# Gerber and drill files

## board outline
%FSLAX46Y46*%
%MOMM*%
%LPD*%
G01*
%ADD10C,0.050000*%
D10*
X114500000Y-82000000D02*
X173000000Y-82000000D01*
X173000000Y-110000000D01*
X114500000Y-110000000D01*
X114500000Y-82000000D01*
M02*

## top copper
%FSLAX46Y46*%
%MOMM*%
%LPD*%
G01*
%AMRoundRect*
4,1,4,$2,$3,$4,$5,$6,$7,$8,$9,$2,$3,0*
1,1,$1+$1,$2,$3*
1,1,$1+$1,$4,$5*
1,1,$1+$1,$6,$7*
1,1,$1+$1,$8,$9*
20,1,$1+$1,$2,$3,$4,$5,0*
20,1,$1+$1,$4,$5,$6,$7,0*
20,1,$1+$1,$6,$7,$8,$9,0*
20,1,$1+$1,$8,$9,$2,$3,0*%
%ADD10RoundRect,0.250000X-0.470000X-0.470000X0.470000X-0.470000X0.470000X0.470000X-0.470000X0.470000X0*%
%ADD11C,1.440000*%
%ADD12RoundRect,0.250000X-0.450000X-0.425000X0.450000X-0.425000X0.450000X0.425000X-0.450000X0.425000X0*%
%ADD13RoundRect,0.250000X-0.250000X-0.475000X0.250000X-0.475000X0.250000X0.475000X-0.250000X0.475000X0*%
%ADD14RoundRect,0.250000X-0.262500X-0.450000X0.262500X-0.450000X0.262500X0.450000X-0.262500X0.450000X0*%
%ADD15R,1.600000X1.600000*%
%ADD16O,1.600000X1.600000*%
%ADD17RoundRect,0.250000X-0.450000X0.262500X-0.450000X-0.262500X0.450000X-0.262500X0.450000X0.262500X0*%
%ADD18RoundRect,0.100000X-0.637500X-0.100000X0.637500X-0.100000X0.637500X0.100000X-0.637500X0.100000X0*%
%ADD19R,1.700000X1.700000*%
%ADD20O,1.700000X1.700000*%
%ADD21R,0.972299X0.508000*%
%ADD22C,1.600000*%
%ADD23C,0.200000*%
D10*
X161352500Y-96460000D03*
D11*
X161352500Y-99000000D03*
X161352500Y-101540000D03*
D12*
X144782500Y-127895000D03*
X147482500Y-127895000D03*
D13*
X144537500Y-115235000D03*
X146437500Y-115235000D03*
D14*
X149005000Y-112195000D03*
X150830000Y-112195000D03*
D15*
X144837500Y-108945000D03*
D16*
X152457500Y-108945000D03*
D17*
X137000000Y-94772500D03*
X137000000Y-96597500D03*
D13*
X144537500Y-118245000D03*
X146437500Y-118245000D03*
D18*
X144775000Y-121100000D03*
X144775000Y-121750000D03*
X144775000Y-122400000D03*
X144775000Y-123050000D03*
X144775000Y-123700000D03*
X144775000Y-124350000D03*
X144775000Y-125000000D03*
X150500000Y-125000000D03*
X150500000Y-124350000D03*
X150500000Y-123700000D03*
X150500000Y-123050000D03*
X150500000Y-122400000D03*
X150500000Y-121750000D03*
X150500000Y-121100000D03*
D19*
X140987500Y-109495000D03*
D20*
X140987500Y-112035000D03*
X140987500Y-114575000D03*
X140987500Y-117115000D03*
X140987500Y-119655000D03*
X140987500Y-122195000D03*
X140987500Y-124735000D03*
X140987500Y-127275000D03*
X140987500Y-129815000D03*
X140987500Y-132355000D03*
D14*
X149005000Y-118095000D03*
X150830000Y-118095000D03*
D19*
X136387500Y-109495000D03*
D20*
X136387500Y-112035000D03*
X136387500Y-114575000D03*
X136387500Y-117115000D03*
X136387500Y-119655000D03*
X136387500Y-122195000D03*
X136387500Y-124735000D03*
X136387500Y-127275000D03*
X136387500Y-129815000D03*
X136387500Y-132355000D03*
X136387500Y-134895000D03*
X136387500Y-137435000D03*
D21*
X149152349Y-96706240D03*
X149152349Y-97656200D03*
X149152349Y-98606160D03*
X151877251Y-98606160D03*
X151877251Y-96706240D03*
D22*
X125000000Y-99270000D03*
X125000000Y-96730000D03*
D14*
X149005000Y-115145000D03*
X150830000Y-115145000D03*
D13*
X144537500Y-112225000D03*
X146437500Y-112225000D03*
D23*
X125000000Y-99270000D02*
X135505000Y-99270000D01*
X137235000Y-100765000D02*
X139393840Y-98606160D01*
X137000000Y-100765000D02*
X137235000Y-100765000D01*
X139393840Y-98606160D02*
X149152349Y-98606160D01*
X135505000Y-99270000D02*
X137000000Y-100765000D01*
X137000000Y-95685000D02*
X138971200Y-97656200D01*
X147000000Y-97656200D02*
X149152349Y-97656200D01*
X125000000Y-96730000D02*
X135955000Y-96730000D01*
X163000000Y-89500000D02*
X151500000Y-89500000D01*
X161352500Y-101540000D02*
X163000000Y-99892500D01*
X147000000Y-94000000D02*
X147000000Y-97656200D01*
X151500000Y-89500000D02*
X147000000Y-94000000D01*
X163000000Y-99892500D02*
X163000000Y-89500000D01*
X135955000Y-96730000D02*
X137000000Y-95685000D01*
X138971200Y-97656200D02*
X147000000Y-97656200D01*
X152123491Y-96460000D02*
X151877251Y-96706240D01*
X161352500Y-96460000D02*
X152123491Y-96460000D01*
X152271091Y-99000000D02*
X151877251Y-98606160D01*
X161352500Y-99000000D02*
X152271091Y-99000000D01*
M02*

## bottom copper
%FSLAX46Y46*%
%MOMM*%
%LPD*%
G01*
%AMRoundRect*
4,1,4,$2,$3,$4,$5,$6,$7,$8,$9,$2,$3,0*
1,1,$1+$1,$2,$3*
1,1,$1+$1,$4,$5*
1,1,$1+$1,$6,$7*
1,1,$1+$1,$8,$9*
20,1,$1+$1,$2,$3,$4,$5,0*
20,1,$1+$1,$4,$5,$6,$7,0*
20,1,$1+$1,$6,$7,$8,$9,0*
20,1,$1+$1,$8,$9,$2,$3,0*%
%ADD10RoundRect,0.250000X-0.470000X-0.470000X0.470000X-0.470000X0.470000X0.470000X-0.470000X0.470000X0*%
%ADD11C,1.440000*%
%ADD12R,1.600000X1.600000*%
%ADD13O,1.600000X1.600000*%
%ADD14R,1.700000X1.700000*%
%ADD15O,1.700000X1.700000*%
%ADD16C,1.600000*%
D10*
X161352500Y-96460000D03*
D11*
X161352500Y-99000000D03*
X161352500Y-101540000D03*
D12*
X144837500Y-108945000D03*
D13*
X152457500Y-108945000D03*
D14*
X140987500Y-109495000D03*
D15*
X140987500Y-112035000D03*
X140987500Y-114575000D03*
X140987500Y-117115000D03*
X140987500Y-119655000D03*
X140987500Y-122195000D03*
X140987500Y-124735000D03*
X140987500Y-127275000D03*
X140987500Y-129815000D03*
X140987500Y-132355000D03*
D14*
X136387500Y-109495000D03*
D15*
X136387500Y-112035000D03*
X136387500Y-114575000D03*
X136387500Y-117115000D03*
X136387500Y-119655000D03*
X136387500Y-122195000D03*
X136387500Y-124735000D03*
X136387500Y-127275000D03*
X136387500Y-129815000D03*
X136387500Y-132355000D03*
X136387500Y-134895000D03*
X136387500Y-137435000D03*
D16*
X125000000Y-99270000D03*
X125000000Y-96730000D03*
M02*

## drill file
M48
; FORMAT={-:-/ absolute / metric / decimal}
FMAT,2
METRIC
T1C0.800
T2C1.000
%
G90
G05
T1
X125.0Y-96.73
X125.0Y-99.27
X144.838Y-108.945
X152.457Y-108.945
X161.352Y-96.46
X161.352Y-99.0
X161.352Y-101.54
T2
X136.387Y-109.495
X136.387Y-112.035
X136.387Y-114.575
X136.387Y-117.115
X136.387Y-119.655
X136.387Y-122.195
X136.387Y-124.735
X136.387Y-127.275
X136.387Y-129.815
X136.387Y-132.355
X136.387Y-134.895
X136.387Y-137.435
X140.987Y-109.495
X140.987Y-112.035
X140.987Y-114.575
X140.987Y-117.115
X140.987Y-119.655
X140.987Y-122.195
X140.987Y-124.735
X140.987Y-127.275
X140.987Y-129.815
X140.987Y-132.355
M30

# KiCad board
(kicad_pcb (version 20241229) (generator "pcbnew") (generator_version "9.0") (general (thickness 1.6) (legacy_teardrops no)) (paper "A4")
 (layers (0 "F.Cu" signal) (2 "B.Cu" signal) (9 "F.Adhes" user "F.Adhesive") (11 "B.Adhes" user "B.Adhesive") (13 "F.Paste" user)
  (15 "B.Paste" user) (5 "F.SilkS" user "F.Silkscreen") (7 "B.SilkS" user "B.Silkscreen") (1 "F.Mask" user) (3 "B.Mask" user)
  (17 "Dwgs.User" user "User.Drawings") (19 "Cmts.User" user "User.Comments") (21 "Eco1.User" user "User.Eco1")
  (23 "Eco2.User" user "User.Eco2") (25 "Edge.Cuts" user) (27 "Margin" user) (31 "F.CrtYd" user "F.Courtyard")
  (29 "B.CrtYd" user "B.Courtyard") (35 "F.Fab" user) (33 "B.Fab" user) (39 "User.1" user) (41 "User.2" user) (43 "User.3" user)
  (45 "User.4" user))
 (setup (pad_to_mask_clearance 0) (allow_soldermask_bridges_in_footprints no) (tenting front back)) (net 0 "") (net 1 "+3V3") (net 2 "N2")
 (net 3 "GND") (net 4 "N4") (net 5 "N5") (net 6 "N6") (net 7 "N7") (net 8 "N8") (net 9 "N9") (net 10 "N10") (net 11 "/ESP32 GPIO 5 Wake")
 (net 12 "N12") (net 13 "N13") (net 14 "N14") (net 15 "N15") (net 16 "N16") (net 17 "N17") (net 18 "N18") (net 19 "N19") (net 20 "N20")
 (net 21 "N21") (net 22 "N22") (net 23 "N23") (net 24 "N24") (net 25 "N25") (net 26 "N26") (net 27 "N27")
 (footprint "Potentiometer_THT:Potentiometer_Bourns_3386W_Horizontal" (layer "F.Cu") (at 161.3525 96.46 -90)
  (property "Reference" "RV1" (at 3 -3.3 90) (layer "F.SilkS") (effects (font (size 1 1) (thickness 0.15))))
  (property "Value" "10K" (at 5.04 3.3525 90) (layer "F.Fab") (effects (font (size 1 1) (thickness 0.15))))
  (pad "1" thru_hole roundrect (at 0 0) (size 1.44 1.44) (drill 0.8) (layers "*.Cu" "*.Mask") (remove_unused_layers no)
   (roundrect_rratio 0.1736111111) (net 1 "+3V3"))
  (pad "2" thru_hole circle (at 2.54 0) (size 1.44 1.44) (drill 0.8) (layers "*.Cu" "*.Mask") (remove_unused_layers no) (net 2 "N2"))
  (pad "3" thru_hole circle (at 5.08 0) (size 1.44 1.44) (drill 0.8) (layers "*.Cu" "*.Mask") (remove_unused_layers no) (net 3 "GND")))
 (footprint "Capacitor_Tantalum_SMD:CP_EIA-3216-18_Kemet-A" (layer "F.Cu") (at 146.1325 127.895)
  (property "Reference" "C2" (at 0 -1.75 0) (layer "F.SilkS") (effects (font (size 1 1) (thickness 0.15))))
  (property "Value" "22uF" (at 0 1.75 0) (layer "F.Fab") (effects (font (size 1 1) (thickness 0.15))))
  (pad "1" smd roundrect (at -1.35 0) (size 1.4 1.35) (layers "F.Cu" "F.Mask" "F.Paste") (roundrect_rratio 0.185185) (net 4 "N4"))
  (pad "2" smd roundrect (at 1.35 0) (size 1.4 1.35) (layers "F.Cu" "F.Mask" "F.Paste") (roundrect_rratio 0.185185) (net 3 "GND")))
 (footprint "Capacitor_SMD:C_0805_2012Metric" (layer "F.Cu") (at 145.4875 115.235)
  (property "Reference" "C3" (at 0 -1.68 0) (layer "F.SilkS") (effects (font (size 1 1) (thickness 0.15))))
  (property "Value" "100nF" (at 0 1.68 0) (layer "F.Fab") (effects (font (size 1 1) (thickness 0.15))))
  (pad "1" smd roundrect (at -0.95 0) (size 1 1.45) (layers "F.Cu" "F.Mask" "F.Paste") (roundrect_rratio 0.25) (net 1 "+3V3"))
  (pad "2" smd roundrect (at 0.95 0) (size 1 1.45) (layers "F.Cu" "F.Mask" "F.Paste") (roundrect_rratio 0.25) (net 3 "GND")))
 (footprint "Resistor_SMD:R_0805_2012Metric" (layer "F.Cu") (at 149.9175 112.195)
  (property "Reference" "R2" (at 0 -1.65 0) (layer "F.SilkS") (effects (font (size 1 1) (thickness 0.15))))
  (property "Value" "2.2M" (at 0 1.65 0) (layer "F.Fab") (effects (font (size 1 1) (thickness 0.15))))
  (pad "1" smd roundrect (at -0.9125 0) (size 1.025 1.4) (layers "F.Cu" "F.Mask" "F.Paste") (roundrect_rratio 0.243902) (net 4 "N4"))
  (pad "2" smd roundrect (at 0.9125 0) (size 1.025 1.4) (layers "F.Cu" "F.Mask" "F.Paste") (roundrect_rratio 0.243902) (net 1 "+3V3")))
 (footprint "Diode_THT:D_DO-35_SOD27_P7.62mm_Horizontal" (layer "F.Cu") (at 144.8375 108.945)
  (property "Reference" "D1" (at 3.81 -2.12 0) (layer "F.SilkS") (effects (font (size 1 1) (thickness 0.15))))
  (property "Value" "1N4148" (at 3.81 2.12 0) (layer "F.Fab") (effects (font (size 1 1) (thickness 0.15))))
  (pad "1" thru_hole rect (at 0 0) (size 1.6 1.6) (drill 0.8) (layers "*.Cu" "*.Mask") (remove_unused_layers no) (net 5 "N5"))
  (pad "2" thru_hole oval (at 7.62 0) (size 1.6 1.6) (drill 0.8) (layers "*.Cu" "*.Mask") (remove_unused_layers no) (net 4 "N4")))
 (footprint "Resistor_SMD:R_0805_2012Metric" (layer "F.Cu") (at 137 95.685 -90)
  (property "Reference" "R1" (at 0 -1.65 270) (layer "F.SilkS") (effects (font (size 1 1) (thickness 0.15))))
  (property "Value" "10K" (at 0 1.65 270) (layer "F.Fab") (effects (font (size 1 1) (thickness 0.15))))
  (pad "1" smd roundrect (at -0.9125 0 270) (size 1.025 1.4) (layers "F.Cu" "F.Mask" "F.Paste") (roundrect_rratio 0.243902) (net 3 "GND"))
  (pad "2" smd roundrect (at 0.9125 0 270) (size 1.025 1.4) (layers "F.Cu" "F.Mask" "F.Paste") (roundrect_rratio 0.243902) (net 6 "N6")))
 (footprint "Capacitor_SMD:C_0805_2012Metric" (layer "F.Cu") (at 145.4875 118.245)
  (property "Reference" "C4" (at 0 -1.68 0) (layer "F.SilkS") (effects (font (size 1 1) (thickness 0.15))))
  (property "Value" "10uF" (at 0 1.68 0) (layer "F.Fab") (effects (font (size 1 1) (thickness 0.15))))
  (pad "1" smd roundrect (at -0.95 0) (size 1 1.45) (layers "F.Cu" "F.Mask" "F.Paste") (roundrect_rratio 0.25) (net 3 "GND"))
  (pad "2" smd roundrect (at 0.95 0) (size 1 1.45) (layers "F.Cu" "F.Mask" "F.Paste") (roundrect_rratio 0.25) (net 1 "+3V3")))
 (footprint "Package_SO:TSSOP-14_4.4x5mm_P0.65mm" (layer "F.Cu") (at 147.6375 123.05)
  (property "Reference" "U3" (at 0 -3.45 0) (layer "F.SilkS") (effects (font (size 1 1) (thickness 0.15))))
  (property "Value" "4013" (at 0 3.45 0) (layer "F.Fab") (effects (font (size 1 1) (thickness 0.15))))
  (pad "1" smd roundrect (at -2.8625 -1.95) (size 1.475 0.4) (layers "F.Cu" "F.Mask" "F.Paste") (roundrect_rratio 0.25) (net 5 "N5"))
  (pad "2" smd roundrect (at -2.8625 -1.3) (size 1.475 0.4) (layers "F.Cu" "F.Mask" "F.Paste") (roundrect_rratio 0.25) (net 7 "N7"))
  (pad "3" smd roundrect (at -2.8625 -0.65) (size 1.475 0.4) (layers "F.Cu" "F.Mask" "F.Paste") (roundrect_rratio 0.25) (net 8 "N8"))
  (pad "4" smd roundrect (at -2.8625 0) (size 1.475 0.4) (layers "F.Cu" "F.Mask" "F.Paste") (roundrect_rratio 0.25) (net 4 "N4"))
  (pad "5" smd roundrect (at -2.8625 0.65) (size 1.475 0.4) (layers "F.Cu" "F.Mask" "F.Paste") (roundrect_rratio 0.25) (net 1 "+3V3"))
  (pad "6" smd roundrect (at -2.8625 1.3) (size 1.475 0.4) (layers "F.Cu" "F.Mask" "F.Paste") (roundrect_rratio 0.25) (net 3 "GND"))
  (pad "7" smd roundrect (at -2.8625 1.95) (size 1.475 0.4) (layers "F.Cu" "F.Mask" "F.Paste") (roundrect_rratio 0.25) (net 3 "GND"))
  (pad "8" smd roundrect (at 2.8625 1.95) (size 1.475 0.4) (layers "F.Cu" "F.Mask" "F.Paste") (roundrect_rratio 0.25) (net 3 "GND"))
  (pad "9" smd roundrect (at 2.8625 1.3) (size 1.475 0.4) (layers "F.Cu" "F.Mask" "F.Paste") (roundrect_rratio 0.25) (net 1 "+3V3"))
  (pad "10" smd roundrect (at 2.8625 0.65) (size 1.475 0.4) (layers "F.Cu" "F.Mask" "F.Paste") (roundrect_rratio 0.25) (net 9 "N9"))
  (pad "11" smd roundrect (at 2.8625 0) (size 1.475 0.4) (layers "F.Cu" "F.Mask" "F.Paste") (roundrect_rratio 0.25) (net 8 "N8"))
  (pad "12" smd roundrect (at 2.8625 -0.65) (size 1.475 0.4) (layers "F.Cu" "F.Mask" "F.Paste") (roundrect_rratio 0.25) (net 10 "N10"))
  (pad "13" smd roundrect (at 2.8625 -1.3) (size 1.475 0.4) (layers "F.Cu" "F.Mask" "F.Paste") (roundrect_rratio 0.25)
   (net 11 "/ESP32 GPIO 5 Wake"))
  (pad "14" smd roundrect (at 2.8625 -1.95) (size 1.475 0.4) (layers "F.Cu" "F.Mask" "F.Paste") (roundrect_rratio 0.25) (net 1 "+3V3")))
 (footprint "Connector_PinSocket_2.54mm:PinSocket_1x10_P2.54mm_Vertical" (layer "F.Cu") (at 140.9875 109.495)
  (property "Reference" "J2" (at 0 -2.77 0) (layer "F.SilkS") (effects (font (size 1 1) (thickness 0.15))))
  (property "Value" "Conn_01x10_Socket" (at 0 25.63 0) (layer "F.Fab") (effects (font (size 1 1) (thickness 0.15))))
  (pad "1" thru_hole rect (at 0 0) (size 1.7 1.7) (drill 1) (layers "*.Cu" "*.Mask") (remove_unused_layers no) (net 1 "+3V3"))
  (pad "2" thru_hole oval (at 0 2.54) (size 1.7 1.7) (drill 1) (layers "*.Cu" "*.Mask") (remove_unused_layers no) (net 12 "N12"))
  (pad "3" thru_hole oval (at 0 5.08) (size 1.7 1.7) (drill 1) (layers "*.Cu" "*.Mask") (remove_unused_layers no) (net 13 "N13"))
  (pad "4" thru_hole oval (at 0 7.62) (size 1.7 1.7) (drill 1) (layers "*.Cu" "*.Mask") (remove_unused_layers no) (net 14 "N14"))
  (pad "5" thru_hole oval (at 0 10.16) (size 1.7 1.7) (drill 1) (layers "*.Cu" "*.Mask") (remove_unused_layers no) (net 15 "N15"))
  (pad "6" thru_hole oval (at 0 12.7) (size 1.7 1.7) (drill 1) (layers "*.Cu" "*.Mask") (remove_unused_layers no) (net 3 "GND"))
  (pad "7" thru_hole oval (at 0 15.24) (size 1.7 1.7) (drill 1) (layers "*.Cu" "*.Mask") (remove_unused_layers no) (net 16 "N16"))
  (pad "8" thru_hole oval (at 0 17.78) (size 1.7 1.7) (drill 1) (layers "*.Cu" "*.Mask") (remove_unused_layers no) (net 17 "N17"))
  (pad "9" thru_hole oval (at 0 20.32) (size 1.7 1.7) (drill 1) (layers "*.Cu" "*.Mask") (remove_unused_layers no) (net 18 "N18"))
  (pad "10" thru_hole oval (at 0 22.86) (size 1.7 1.7) (drill 1) (layers "*.Cu" "*.Mask") (remove_unused_layers no) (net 3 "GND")))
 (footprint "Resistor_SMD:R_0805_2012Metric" (layer "F.Cu") (at 149.9175 118.095)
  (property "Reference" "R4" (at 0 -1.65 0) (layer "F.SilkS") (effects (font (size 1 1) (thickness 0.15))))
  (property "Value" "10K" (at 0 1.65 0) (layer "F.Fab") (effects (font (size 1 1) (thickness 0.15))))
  (pad "1" smd roundrect (at -0.9125 0) (size 1.025 1.4) (layers "F.Cu" "F.Mask" "F.Paste") (roundrect_rratio 0.243902) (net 9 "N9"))
  (pad "2" smd roundrect (at 0.9125 0) (size 1.025 1.4) (layers "F.Cu" "F.Mask" "F.Paste") (roundrect_rratio 0.243902) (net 5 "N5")))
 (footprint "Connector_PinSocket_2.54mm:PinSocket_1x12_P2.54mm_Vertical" (layer "F.Cu") (at 136.3875 109.495)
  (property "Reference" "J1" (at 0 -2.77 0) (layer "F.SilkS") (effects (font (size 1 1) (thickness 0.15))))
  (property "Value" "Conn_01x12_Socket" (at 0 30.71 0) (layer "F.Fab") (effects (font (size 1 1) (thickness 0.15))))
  (pad "1" thru_hole rect (at 0 0) (size 1.7 1.7) (drill 1) (layers "*.Cu" "*.Mask") (remove_unused_layers no) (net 3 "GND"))
  (pad "2" thru_hole oval (at 0 2.54) (size 1.7 1.7) (drill 1) (layers "*.Cu" "*.Mask") (remove_unused_layers no) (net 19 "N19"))
  (pad "3" thru_hole oval (at 0 5.08) (size 1.7 1.7) (drill 1) (layers "*.Cu" "*.Mask") (remove_unused_layers no)
   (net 11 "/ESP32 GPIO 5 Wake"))
  (pad "4" thru_hole oval (at 0 7.62) (size 1.7 1.7) (drill 1) (layers "*.Cu" "*.Mask") (remove_unused_layers no) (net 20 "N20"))
  (pad "5" thru_hole oval (at 0 10.16) (size 1.7 1.7) (drill 1) (layers "*.Cu" "*.Mask") (remove_unused_layers no) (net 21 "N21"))
  (pad "6" thru_hole oval (at 0 12.7) (size 1.7 1.7) (drill 1) (layers "*.Cu" "*.Mask") (remove_unused_layers no) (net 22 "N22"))
  (pad "7" thru_hole oval (at 0 15.24) (size 1.7 1.7) (drill 1) (layers "*.Cu" "*.Mask") (remove_unused_layers no) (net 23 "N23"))
  (pad "8" thru_hole oval (at 0 17.78) (size 1.7 1.7) (drill 1) (layers "*.Cu" "*.Mask") (remove_unused_layers no) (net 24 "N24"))
  (pad "9" thru_hole oval (at 0 20.32) (size 1.7 1.7) (drill 1) (layers "*.Cu" "*.Mask") (remove_unused_layers no) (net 3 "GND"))
  (pad "10" thru_hole oval (at 0 22.86) (size 1.7 1.7) (drill 1) (layers "*.Cu" "*.Mask") (remove_unused_layers no) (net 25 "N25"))
  (pad "11" thru_hole oval (at 0 25.4) (size 1.7 1.7) (drill 1) (layers "*.Cu" "*.Mask") (remove_unused_layers no) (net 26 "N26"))
  (pad "12" thru_hole oval (at 0 27.94) (size 1.7 1.7) (drill 1) (layers "*.Cu" "*.Mask") (remove_unused_layers no) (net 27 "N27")))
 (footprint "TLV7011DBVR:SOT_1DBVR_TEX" (layer "F.Cu") (at 150.5148 97.6562)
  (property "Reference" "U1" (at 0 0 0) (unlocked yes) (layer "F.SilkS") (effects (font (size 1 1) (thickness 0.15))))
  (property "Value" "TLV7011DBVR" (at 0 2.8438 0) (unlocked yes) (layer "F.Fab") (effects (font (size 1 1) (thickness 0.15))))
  (pad "1" smd rect (at -1.362451 -0.94996) (size 0.972299 0.508) (layers "F.Cu" "F.Mask" "F.Paste") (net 8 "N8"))
  (pad "2" smd rect (at -1.362451 0) (size 0.972299 0.508) (layers "F.Cu" "F.Mask" "F.Paste") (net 3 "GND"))
  (pad "3" smd rect (at -1.362451 0.94996) (size 0.972299 0.508) (layers "F.Cu" "F.Mask" "F.Paste") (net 6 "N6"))
  (pad "4" smd rect (at 1.362451 0.94996) (size 0.972299 0.508) (layers "F.Cu" "F.Mask" "F.Paste") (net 2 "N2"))
  (pad "5" smd rect (at 1.362451 -0.94996) (size 0.972299 0.508) (layers "F.Cu" "F.Mask" "F.Paste") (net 1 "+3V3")))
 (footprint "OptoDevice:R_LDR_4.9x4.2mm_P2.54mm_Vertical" (layer "F.Cu") (at 125 99.27 90)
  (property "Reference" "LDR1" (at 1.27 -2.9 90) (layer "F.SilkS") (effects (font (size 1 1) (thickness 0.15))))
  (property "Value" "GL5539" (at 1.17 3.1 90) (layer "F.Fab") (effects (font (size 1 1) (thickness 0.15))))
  (pad "1" thru_hole circle (at 0 0 90) (size 1.6 1.6) (drill 0.8) (layers "*.Cu" "*.Mask") (remove_unused_layers no) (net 6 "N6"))
  (pad "2" thru_hole circle (at 2.54 0 90) (size 1.6 1.6) (drill 0.8) (layers "*.Cu" "*.Mask") (remove_unused_layers no) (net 1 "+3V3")))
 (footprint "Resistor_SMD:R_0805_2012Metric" (layer "F.Cu") (at 149.9175 115.145)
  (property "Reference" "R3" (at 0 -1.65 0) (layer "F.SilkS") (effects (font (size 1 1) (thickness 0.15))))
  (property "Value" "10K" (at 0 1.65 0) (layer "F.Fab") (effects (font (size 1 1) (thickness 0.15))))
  (pad "1" smd roundrect (at -0.9125 0) (size 1.025 1.4) (layers "F.Cu" "F.Mask" "F.Paste") (roundrect_rratio 0.243902) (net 8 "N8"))
  (pad "2" smd roundrect (at 0.9125 0) (size 1.025 1.4) (layers "F.Cu" "F.Mask" "F.Paste") (roundrect_rratio 0.243902) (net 3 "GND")))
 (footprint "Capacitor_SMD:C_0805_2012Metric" (layer "F.Cu") (at 145.4875 112.225)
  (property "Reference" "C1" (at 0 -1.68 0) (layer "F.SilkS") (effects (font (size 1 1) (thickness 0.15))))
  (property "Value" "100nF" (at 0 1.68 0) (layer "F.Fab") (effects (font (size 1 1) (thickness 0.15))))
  (pad "1" smd roundrect (at -0.95 0) (size 1 1.45) (layers "F.Cu" "F.Mask" "F.Paste") (roundrect_rratio 0.25) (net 9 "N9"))
  (pad "2" smd roundrect (at 0.95 0) (size 1 1.45) (layers "F.Cu" "F.Mask" "F.Paste") (roundrect_rratio 0.25) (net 3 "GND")))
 (gr_rect (start 114.5 82) (end 173 110) (stroke (width 0.05) (type default)) (fill no) (layer "Edge.Cuts"))
 (segment (start 125 99.27) (end 135.505 99.27) (width 0.2) (layer "F.Cu") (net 6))
 (segment (start 137.235 100.765) (end 139.39384 98.60616) (width 0.2) (layer "F.Cu") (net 6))
 (segment (start 137 100.765) (end 137.235 100.765) (width 0.2) (layer "F.Cu") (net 6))
 (segment (start 139.39384 98.60616) (end 149.152349 98.60616) (width 0.2) (layer "F.Cu") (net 6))
 (segment (start 135.505 99.27) (end 137 100.765) (width 0.2) (layer "F.Cu") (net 6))
 (segment (start 137 95.685) (end 138.9712 97.6562) (width 0.2) (layer "F.Cu") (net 3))
 (segment (start 147 97.6562) (end 149.152349 97.6562) (width 0.2) (layer "F.Cu") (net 3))
 (segment (start 125 96.73) (end 135.955 96.73) (width 0.2) (layer "F.Cu") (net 3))
 (segment (start 163 89.5) (end 151.5 89.5) (width 0.2) (layer "F.Cu") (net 3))
 (segment (start 161.3525 101.54) (end 163 99.8925) (width 0.2) (layer "F.Cu") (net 3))
 (segment (start 147 94) (end 147 97.6562) (width 0.2) (layer "F.Cu") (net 3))
 (segment (start 151.5 89.5) (end 147 94) (width 0.2) (layer "F.Cu") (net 3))
 (segment (start 163 99.8925) (end 163 89.5) (width 0.2) (layer "F.Cu") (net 3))
 (segment (start 135.955 96.73) (end 137 95.685) (width 0.2) (layer "F.Cu") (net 3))
 (segment (start 138.9712 97.6562) (end 147 97.6562) (width 0.2) (layer "F.Cu") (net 3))
 (segment (start 152.123491 96.46) (end 151.877251 96.70624) (width 0.2) (layer "F.Cu") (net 1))
 (segment (start 161.3525 96.46) (end 152.123491 96.46) (width 0.2) (layer "F.Cu") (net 1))
 (segment (start 152.271091 99) (end 151.877251 98.60616) (width 0.2) (layer "F.Cu") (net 2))
 (segment (start 161.3525 99) (end 152.271091 99) (width 0.2) (layer "F.Cu") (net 2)))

